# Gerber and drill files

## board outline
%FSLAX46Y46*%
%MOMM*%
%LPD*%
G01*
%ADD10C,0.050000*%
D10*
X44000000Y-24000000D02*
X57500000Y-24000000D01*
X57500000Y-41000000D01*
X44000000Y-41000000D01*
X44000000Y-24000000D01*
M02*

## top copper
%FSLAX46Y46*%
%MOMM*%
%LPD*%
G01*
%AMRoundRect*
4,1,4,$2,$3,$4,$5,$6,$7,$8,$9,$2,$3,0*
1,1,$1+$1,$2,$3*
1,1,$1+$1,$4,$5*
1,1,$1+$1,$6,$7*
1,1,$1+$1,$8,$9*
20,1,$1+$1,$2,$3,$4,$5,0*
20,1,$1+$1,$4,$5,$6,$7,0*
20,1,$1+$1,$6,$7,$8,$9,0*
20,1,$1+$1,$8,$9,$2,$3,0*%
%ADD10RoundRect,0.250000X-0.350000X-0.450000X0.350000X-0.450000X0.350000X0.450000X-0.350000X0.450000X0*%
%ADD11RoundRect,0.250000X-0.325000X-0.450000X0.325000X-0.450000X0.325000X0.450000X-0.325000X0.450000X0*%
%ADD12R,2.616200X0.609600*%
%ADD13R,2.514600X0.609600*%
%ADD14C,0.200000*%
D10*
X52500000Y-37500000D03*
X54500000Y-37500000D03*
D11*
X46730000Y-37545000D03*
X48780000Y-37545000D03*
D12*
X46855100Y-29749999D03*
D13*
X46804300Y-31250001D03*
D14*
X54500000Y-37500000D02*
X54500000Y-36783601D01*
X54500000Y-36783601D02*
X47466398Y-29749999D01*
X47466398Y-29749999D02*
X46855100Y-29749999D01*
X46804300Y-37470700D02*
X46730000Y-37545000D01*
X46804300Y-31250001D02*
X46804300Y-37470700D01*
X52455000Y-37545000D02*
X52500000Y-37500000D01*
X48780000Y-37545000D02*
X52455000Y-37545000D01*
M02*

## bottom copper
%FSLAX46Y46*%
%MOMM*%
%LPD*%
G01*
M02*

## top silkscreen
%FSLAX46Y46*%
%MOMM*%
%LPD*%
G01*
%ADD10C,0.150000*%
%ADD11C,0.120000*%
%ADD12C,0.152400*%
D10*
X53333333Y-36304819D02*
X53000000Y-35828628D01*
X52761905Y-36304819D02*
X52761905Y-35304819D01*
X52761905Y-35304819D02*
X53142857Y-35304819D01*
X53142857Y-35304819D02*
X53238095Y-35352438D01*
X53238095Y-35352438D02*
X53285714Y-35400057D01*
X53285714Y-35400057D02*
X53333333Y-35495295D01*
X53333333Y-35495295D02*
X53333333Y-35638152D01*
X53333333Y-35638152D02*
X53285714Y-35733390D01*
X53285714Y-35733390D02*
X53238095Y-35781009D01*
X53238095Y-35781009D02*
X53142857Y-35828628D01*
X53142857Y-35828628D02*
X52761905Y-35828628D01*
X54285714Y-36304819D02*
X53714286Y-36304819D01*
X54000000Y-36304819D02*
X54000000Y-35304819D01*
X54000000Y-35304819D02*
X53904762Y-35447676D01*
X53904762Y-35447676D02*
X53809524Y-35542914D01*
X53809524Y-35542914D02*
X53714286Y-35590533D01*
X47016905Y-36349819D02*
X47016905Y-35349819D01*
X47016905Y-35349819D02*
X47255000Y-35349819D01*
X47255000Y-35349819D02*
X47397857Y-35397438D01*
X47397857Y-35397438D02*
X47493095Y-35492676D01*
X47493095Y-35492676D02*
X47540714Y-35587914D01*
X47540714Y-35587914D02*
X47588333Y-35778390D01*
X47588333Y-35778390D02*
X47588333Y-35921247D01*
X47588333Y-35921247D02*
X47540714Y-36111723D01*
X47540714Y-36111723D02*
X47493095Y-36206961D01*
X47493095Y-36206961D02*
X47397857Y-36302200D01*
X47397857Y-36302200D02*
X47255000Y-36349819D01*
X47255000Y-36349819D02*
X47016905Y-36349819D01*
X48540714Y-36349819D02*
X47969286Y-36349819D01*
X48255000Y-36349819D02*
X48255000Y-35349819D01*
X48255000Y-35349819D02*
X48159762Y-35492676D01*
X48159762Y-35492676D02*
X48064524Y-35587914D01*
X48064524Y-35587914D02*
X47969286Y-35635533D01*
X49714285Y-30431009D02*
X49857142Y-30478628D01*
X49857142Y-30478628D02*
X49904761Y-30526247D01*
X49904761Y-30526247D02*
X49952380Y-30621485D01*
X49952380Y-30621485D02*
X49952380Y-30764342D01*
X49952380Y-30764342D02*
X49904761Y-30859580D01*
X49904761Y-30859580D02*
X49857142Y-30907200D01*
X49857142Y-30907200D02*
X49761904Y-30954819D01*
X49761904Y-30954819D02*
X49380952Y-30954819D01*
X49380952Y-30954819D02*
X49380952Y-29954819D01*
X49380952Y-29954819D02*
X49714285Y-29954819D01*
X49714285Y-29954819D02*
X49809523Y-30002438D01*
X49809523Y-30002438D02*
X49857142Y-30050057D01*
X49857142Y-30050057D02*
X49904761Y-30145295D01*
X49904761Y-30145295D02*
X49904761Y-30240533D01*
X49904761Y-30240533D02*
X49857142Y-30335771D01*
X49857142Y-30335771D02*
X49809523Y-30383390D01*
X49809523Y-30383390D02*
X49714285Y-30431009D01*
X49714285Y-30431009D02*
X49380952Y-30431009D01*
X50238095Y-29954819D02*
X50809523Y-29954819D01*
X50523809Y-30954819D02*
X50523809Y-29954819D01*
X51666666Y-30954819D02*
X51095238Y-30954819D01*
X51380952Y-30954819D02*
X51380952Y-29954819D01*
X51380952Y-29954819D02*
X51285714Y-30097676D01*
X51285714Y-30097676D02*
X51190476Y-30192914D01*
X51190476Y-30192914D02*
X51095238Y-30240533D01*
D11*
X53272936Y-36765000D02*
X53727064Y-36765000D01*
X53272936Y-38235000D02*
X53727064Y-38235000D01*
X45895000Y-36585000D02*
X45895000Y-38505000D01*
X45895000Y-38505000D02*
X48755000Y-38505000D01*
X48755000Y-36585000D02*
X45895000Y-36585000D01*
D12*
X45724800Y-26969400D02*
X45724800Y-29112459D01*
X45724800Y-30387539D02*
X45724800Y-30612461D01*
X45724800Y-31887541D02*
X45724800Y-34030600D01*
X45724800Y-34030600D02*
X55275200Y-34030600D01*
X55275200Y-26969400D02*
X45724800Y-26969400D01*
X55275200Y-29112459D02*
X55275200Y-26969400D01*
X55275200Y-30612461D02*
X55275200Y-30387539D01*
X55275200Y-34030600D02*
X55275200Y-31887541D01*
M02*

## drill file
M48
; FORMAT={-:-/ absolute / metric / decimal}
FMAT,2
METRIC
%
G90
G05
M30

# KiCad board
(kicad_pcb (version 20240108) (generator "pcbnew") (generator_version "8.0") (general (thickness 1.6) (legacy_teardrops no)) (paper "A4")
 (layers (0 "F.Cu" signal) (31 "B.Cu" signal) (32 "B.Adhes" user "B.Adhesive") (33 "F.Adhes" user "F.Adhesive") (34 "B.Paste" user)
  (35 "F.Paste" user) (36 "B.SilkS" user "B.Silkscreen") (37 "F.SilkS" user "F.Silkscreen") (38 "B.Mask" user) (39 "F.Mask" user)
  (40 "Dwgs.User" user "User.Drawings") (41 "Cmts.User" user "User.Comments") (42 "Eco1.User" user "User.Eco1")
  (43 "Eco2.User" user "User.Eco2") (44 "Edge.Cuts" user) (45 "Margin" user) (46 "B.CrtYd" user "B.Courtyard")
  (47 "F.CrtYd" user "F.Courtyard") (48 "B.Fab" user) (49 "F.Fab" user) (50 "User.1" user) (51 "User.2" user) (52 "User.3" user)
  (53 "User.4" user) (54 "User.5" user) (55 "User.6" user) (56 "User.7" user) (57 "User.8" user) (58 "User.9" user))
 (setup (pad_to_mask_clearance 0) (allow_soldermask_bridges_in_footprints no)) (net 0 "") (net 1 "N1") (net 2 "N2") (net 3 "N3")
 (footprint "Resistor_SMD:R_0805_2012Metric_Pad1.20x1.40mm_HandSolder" (layer "F.Cu") (at 53.5 37.5)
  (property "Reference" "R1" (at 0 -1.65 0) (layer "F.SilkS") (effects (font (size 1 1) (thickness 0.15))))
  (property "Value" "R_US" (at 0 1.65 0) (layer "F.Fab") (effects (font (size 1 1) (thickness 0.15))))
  (fp_line (start -0.227064 -0.735) (end 0.227064 -0.735) (stroke (width 0.12) (type solid)) (layer "F.SilkS"))
  (fp_line (start -0.227064 0.735) (end 0.227064 0.735) (stroke (width 0.12) (type solid)) (layer "F.SilkS"))
  (pad "1" smd roundrect (at -1 0) (size 1.2 1.4) (layers "F.Cu" "F.Paste" "F.Mask") (roundrect_rratio 0.208333) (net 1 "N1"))
  (pad "2" smd roundrect (at 1 0) (size 1.2 1.4) (layers "F.Cu" "F.Paste" "F.Mask") (roundrect_rratio 0.208333) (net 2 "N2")))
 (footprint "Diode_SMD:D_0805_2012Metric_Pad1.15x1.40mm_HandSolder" (layer "F.Cu") (at 47.755 37.545)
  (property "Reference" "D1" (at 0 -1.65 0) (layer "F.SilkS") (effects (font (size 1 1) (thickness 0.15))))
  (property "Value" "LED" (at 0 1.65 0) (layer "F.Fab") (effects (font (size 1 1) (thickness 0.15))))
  (fp_line (start -1.86 -0.96) (end -1.86 0.96) (stroke (width 0.12) (type solid)) (layer "F.SilkS"))
  (fp_line (start -1.86 0.96) (end 1 0.96) (stroke (width 0.12) (type solid)) (layer "F.SilkS"))
  (fp_line (start 1 -0.96) (end -1.86 -0.96) (stroke (width 0.12) (type solid)) (layer "F.SilkS"))
  (pad "1" smd roundrect (at -1.025 0) (size 1.15 1.4) (layers "F.Cu" "F.Paste" "F.Mask") (roundrect_rratio 0.217391) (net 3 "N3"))
  (pad "2" smd roundrect (at 1.025 0) (size 1.15 1.4) (layers "F.Cu" "F.Paste" "F.Mask") (roundrect_rratio 0.217391) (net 1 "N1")))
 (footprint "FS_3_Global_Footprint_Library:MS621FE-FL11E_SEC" (layer "F.Cu") (at 50.5 30.5)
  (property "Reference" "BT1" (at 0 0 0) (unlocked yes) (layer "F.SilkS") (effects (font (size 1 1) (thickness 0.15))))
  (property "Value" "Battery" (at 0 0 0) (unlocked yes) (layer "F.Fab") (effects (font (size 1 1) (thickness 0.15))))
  (fp_line (start -4.7752 -3.5306) (end -4.7752 -1.387541) (stroke (width 0.1524) (type solid)) (layer "F.SilkS"))
  (fp_line (start -4.7752 -0.112461) (end -4.7752 0.112461) (stroke (width 0.1524) (type solid)) (layer "F.SilkS"))
  (fp_line (start -4.7752 1.387541) (end -4.7752 3.5306) (stroke (width 0.1524) (type solid)) (layer "F.SilkS"))
  (fp_line (start -4.7752 3.5306) (end 4.7752 3.5306) (stroke (width 0.1524) (type solid)) (layer "F.SilkS"))
  (fp_line (start 4.7752 -3.5306) (end -4.7752 -3.5306) (stroke (width 0.1524) (type solid)) (layer "F.SilkS"))
  (fp_line (start 4.7752 -1.387541) (end 4.7752 -3.5306) (stroke (width 0.1524) (type solid)) (layer "F.SilkS"))
  (fp_line (start 4.7752 0.112461) (end 4.7752 -0.112461) (stroke (width 0.1524) (type solid)) (layer "F.SilkS"))
  (fp_line (start 4.7752 3.5306) (end 4.7752 1.387541) (stroke (width 0.1524) (type solid)) (layer "F.SilkS"))
  (pad "1" smd rect (at -3.6449 -0.750001) (size 2.6162 0.6096) (layers "F.Cu" "F.Paste" "F.Mask") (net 2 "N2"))
  (pad "2" smd rect (at -3.6957 0.750001) (size 2.5146 0.6096) (layers "F.Cu" "F.Paste" "F.Mask") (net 3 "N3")))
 (gr_rect (start 44 24) (end 57.5 41) (stroke (width 0.05) (type default)) (fill none) (layer "Edge.Cuts"))
 (segment (start 54.5 37.5) (end 54.5 36.783601) (width 0.2) (layer "F.Cu") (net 2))
 (segment (start 54.5 36.783601) (end 47.466398 29.749999) (width 0.2) (layer "F.Cu") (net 2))
 (segment (start 47.466398 29.749999) (end 46.8551 29.749999) (width 0.2) (layer "F.Cu") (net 2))
 (segment (start 46.8043 37.4707) (end 46.73 37.545) (width 0.2) (layer "F.Cu") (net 3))
 (segment (start 46.8043 31.250001) (end 46.8043 37.4707) (width 0.2) (layer "F.Cu") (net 3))
 (segment (start 52.455 37.545) (end 52.5 37.5) (width 0.2) (layer "F.Cu") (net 1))
 (segment (start 48.78 37.545) (end 52.455 37.545) (width 0.2) (layer "F.Cu") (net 1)))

